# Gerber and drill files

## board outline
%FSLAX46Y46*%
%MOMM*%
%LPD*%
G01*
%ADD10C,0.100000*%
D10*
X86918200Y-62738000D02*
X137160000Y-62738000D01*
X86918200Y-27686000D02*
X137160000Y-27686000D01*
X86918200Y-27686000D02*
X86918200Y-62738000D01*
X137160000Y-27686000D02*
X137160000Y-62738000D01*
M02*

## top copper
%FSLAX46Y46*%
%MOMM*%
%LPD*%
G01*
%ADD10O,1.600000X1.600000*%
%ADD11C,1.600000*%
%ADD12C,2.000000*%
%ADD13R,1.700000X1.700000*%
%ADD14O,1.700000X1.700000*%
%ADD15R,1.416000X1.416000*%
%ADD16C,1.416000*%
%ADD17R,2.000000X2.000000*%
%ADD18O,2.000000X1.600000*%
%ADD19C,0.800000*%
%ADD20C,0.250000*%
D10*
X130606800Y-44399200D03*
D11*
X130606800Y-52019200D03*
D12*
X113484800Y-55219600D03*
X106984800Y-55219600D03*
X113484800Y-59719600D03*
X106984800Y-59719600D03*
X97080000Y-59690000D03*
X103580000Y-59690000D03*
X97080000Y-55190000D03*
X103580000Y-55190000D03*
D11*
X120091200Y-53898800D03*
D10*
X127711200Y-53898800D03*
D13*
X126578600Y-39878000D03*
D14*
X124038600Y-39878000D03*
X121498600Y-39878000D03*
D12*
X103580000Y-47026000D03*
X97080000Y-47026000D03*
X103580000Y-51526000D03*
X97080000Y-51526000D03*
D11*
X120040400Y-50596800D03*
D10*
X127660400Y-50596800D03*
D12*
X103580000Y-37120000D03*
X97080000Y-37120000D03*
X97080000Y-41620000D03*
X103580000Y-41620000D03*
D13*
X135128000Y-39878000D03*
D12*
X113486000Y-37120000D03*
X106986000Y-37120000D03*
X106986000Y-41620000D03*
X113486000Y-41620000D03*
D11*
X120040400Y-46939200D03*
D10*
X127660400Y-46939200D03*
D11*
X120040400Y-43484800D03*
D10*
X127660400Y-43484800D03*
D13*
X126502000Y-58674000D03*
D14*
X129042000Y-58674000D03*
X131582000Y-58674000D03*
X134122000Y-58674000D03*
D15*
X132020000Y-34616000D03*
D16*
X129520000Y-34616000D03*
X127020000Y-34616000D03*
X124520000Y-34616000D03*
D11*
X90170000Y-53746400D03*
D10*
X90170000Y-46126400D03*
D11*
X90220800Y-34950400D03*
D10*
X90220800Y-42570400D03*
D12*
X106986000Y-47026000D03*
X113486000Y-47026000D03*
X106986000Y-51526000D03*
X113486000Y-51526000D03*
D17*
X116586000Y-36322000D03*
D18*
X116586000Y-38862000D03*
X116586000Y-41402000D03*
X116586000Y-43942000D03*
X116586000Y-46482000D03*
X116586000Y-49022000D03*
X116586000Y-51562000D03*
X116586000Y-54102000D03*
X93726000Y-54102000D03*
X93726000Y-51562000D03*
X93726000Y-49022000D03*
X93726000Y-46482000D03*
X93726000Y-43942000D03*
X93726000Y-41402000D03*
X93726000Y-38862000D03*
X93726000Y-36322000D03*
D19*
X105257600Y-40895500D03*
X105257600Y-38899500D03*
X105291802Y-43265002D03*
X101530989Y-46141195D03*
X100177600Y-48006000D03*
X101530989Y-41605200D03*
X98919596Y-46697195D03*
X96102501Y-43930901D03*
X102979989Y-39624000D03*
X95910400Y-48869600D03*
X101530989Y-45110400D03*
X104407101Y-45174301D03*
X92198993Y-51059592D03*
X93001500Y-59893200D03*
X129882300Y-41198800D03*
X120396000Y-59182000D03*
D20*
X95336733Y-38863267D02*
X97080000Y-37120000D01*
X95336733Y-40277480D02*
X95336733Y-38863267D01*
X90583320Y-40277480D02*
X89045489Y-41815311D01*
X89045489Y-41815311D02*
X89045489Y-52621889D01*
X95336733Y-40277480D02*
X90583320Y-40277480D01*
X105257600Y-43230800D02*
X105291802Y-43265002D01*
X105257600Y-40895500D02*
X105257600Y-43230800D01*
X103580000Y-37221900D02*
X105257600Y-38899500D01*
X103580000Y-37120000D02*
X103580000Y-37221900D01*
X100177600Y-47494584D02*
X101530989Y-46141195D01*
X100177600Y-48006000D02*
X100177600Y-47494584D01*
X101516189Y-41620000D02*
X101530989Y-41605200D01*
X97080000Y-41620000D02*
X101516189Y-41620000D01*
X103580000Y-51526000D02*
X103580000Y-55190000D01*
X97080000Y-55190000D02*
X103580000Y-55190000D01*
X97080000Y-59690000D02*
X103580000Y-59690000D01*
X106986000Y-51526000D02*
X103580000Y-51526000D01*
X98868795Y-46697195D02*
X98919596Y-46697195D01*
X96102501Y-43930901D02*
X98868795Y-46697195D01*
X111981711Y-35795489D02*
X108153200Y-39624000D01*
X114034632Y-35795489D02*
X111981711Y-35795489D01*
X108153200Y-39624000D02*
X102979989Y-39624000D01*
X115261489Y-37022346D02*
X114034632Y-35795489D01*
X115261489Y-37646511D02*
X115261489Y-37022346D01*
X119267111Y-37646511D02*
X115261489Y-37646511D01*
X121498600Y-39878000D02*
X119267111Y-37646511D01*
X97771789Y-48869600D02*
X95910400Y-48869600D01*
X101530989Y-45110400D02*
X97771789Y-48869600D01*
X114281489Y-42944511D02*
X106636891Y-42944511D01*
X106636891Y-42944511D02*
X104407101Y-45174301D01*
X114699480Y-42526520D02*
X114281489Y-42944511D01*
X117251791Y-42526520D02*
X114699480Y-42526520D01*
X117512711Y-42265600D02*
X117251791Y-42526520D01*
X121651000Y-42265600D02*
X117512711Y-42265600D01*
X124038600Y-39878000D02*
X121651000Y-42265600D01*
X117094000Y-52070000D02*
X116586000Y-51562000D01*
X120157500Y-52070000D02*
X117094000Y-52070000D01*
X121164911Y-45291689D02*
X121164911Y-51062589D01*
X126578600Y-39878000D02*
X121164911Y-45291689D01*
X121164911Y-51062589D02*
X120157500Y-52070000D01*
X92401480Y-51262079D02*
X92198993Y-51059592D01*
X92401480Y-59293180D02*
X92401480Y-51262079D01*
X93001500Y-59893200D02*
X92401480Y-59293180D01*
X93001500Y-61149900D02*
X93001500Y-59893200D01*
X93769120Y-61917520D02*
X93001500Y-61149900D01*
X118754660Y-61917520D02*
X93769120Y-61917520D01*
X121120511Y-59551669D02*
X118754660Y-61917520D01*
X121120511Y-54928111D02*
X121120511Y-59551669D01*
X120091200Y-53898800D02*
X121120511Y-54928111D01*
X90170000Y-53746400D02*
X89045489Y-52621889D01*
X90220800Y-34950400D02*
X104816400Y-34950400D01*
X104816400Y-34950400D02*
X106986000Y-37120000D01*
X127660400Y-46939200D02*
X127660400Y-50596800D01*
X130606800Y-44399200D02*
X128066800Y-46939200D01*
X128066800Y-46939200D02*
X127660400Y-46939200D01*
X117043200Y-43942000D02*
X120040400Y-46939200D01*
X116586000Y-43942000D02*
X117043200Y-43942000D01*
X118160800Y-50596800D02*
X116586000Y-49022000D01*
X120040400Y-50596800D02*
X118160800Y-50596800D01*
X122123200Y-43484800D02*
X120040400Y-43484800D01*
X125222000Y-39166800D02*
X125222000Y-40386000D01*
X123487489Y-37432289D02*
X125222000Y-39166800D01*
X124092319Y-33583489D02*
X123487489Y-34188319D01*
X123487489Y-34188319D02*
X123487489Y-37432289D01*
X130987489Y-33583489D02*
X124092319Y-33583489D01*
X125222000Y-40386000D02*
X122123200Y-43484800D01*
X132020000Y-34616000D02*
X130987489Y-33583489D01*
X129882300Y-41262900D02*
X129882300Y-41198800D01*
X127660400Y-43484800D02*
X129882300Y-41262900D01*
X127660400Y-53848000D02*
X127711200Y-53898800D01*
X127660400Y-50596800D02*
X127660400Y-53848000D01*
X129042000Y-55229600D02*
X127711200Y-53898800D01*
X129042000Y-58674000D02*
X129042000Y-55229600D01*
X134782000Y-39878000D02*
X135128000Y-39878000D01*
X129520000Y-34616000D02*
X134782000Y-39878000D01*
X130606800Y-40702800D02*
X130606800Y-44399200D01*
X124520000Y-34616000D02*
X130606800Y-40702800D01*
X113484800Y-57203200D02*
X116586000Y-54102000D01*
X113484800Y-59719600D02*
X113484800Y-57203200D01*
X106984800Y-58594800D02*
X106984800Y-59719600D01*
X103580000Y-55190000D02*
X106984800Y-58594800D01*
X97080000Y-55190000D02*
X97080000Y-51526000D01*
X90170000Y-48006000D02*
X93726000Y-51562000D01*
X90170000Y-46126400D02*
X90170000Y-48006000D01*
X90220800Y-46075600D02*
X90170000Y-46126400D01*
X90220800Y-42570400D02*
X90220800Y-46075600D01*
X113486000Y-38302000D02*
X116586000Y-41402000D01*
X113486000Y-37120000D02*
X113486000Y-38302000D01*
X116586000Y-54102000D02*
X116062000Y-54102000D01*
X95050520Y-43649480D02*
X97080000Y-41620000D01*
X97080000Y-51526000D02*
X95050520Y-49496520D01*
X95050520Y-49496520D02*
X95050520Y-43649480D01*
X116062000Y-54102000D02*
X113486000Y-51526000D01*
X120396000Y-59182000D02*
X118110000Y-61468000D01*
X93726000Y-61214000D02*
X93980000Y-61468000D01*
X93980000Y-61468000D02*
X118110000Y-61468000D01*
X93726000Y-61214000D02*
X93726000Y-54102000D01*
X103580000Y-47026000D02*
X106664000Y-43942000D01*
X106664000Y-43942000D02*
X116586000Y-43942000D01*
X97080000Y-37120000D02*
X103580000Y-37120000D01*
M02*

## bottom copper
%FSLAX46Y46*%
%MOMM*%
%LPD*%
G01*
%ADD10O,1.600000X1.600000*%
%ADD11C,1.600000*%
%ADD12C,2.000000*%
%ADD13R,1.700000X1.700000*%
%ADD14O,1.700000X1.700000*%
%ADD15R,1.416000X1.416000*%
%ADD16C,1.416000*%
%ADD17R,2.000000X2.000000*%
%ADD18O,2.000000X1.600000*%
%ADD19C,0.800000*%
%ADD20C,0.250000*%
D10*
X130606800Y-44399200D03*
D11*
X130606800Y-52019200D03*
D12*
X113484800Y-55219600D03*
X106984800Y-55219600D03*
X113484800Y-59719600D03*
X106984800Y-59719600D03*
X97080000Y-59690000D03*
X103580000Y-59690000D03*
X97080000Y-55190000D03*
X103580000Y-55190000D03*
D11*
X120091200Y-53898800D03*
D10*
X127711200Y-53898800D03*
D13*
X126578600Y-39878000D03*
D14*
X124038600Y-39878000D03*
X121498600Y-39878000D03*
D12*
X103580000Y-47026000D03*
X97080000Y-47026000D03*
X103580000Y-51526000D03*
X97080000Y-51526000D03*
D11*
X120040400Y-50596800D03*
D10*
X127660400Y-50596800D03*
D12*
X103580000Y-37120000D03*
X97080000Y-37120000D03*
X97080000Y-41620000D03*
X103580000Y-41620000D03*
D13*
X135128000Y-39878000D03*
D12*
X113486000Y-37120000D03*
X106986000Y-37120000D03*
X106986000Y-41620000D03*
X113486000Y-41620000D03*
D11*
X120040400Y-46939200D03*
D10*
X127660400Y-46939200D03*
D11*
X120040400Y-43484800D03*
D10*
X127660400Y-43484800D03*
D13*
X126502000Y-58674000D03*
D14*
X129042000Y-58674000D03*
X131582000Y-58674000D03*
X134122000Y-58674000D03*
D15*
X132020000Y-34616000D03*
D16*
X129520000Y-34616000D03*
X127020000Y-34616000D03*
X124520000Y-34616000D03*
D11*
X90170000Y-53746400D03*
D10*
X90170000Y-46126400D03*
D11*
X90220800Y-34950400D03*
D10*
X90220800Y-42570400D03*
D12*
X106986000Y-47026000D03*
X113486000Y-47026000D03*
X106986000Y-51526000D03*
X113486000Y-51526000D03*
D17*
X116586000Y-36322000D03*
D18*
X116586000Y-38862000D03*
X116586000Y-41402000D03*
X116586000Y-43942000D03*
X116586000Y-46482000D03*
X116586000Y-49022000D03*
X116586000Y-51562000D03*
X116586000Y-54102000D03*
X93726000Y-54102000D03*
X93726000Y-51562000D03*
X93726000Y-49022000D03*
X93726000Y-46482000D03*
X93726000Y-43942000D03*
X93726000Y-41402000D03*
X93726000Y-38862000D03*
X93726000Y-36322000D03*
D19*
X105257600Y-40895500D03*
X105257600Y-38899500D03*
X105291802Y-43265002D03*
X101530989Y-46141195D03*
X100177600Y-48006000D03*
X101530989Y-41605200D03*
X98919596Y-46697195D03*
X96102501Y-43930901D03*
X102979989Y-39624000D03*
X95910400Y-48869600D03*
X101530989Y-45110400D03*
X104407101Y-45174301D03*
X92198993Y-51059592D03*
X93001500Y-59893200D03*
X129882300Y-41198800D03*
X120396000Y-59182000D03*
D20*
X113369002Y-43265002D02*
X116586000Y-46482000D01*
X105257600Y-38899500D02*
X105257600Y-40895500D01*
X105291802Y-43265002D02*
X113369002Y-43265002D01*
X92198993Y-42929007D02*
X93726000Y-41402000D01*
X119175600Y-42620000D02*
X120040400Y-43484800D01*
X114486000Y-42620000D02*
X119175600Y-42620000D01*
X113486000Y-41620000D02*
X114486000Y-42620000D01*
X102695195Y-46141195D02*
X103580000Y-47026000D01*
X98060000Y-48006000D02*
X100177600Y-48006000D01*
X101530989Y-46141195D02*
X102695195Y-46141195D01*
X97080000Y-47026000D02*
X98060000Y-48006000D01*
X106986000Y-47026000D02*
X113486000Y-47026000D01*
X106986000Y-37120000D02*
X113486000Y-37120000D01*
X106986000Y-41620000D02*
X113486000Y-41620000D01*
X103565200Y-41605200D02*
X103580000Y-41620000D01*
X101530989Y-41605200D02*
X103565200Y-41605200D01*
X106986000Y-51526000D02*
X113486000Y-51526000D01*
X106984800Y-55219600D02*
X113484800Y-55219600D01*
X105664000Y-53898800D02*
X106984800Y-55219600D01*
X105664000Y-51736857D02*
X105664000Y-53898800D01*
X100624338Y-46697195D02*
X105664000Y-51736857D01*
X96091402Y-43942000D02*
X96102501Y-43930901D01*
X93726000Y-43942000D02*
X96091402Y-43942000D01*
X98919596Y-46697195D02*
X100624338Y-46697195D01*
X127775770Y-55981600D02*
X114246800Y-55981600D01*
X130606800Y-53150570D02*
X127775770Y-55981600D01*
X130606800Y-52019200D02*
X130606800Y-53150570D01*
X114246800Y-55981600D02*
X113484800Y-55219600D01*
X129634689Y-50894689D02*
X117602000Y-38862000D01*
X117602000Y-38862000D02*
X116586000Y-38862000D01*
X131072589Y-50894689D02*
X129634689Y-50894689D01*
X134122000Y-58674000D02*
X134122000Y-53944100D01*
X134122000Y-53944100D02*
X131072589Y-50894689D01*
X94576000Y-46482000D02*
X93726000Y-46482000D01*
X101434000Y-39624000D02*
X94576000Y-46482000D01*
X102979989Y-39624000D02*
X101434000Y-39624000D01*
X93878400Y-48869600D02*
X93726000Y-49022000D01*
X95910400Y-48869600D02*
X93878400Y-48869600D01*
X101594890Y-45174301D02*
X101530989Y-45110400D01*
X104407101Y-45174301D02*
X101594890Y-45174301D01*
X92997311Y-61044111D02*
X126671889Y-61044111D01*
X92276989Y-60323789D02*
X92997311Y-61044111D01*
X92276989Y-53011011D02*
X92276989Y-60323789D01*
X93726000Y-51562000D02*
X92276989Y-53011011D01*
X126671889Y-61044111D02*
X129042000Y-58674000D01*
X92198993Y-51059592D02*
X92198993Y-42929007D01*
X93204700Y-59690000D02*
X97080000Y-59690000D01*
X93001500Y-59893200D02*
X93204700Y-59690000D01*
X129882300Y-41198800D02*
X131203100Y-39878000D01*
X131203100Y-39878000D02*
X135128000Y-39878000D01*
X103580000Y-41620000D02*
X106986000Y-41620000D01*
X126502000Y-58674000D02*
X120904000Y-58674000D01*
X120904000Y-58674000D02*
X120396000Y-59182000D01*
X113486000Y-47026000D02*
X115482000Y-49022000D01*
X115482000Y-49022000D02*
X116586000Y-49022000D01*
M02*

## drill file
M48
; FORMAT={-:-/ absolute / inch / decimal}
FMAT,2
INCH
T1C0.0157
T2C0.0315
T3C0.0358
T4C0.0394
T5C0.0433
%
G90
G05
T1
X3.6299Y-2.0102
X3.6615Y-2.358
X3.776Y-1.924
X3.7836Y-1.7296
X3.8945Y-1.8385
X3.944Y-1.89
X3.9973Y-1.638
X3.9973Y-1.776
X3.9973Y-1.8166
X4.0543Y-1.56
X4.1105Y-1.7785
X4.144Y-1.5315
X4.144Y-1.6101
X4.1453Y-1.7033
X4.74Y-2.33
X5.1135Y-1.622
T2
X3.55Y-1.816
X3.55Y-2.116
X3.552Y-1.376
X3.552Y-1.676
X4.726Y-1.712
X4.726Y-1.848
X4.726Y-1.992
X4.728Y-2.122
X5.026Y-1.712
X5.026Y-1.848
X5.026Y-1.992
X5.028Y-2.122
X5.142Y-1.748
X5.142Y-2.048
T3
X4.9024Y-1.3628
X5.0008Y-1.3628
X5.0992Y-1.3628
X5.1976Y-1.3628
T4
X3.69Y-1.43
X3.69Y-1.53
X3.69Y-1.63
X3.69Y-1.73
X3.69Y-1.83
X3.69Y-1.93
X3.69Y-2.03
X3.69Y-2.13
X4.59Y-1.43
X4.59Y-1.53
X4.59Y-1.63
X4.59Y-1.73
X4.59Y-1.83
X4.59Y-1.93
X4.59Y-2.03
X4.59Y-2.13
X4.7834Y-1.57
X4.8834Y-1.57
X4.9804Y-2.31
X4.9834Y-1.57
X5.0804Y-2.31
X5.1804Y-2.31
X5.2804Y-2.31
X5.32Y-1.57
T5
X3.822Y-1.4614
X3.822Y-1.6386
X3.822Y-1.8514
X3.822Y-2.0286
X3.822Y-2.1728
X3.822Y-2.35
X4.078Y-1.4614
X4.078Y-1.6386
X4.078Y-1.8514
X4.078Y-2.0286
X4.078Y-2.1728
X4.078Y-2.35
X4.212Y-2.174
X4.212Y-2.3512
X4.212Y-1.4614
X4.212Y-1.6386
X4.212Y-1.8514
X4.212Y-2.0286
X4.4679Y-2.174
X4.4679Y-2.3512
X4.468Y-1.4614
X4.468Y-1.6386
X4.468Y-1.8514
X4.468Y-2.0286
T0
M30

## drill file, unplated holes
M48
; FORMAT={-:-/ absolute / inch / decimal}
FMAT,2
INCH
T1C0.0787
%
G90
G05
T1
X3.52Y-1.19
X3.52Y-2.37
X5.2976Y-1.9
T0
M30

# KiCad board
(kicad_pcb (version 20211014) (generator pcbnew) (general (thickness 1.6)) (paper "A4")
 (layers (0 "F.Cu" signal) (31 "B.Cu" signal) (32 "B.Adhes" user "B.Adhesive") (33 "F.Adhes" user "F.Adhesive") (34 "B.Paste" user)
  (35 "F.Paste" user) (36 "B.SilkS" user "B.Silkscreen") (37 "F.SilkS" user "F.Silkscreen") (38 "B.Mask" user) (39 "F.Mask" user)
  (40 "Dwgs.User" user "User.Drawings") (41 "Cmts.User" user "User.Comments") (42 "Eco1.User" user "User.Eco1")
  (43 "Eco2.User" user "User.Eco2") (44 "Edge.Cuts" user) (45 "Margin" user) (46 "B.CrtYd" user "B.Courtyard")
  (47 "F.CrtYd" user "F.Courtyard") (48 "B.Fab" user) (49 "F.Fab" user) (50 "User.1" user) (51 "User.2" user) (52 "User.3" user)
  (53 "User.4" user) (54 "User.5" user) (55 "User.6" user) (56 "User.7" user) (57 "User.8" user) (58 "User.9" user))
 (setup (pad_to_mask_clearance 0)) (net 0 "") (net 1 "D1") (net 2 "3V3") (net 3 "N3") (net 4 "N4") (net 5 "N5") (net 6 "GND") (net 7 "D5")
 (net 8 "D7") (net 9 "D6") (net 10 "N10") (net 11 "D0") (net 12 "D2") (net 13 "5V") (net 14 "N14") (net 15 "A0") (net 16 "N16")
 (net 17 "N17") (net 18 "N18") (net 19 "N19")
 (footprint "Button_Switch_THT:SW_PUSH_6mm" (layer "F.Cu") (at 103.58 59.69 180)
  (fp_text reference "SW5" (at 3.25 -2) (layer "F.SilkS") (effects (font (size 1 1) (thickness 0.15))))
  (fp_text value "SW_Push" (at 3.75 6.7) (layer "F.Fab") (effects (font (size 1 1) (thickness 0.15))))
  (pad "1" thru_hole circle (at 0 0 270) (size 2 2) (drill 1.1) (layers *.Cu *.Mask) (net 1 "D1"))
  (pad "1" thru_hole circle (at 6.5 0 270) (size 2 2) (drill 1.1) (layers *.Cu *.Mask) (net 1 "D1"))
  (pad "2" thru_hole circle (at 6.5 4.5 270) (size 2 2) (drill 1.1) (layers *.Cu *.Mask) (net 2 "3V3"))
  (pad "2" thru_hole circle (at 0 4.5 270) (size 2 2) (drill 1.1) (layers *.Cu *.Mask) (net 2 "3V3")))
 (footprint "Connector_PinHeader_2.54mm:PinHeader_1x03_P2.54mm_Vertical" (layer "F.Cu") (at 126.5786 39.878 -90)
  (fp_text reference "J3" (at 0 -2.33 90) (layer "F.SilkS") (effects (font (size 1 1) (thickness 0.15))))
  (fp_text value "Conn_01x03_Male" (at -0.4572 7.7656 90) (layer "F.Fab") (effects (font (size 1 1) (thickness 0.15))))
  (pad "1" thru_hole rect (at 0 0 270) (size 1.7 1.7) (drill 1) (layers *.Cu *.Mask) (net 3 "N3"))
  (pad "2" thru_hole oval (at 0 2.54 270) (size 1.7 1.7) (drill 1) (layers *.Cu *.Mask) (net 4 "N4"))
  (pad "3" thru_hole oval (at 0 5.08 270) (size 1.7 1.7) (drill 1) (layers *.Cu *.Mask) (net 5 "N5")))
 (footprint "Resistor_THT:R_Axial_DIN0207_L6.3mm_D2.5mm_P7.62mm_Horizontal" (layer "F.Cu") (at 120.0912 53.8988)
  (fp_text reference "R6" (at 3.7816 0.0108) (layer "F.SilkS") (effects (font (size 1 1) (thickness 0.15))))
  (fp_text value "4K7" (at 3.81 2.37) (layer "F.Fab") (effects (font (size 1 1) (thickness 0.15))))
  (pad "1" thru_hole circle (at 0 0) (size 1.6 1.6) (drill 0.8) (layers *.Cu *.Mask) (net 1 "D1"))
  (pad "2" thru_hole oval (at 7.62 0) (size 1.6 1.6) (drill 0.8) (layers *.Cu *.Mask) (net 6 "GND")))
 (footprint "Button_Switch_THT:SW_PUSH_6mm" (layer "F.Cu") (at 97.08 47.026)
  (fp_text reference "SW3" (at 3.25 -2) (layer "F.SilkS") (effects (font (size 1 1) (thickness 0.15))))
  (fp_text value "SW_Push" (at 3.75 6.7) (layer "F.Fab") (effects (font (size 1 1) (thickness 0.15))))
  (pad "1" thru_hole circle (at 6.5 0 90) (size 2 2) (drill 1.1) (layers *.Cu *.Mask) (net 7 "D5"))
  (pad "1" thru_hole circle (at 0 0 90) (size 2 2) (drill 1.1) (layers *.Cu *.Mask) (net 7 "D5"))
  (pad "2" thru_hole circle (at 6.5 4.5 90) (size 2 2) (drill 1.1) (layers *.Cu *.Mask) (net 2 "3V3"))
  (pad "2" thru_hole circle (at 0 4.5 90) (size 2 2) (drill 1.1) (layers *.Cu *.Mask) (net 2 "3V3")))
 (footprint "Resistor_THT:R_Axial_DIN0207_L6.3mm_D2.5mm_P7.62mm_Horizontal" (layer "F.Cu") (at 120.0404 50.5968)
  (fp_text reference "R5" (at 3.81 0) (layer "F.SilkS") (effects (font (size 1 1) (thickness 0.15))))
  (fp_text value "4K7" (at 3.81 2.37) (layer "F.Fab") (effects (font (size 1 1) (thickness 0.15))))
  (pad "1" thru_hole circle (at 0 0) (size 1.6 1.6) (drill 0.8) (layers *.Cu *.Mask) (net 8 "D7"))
  (pad "2" thru_hole oval (at 7.62 0) (size 1.6 1.6) (drill 0.8) (layers *.Cu *.Mask) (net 6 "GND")))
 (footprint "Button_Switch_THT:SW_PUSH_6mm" (layer "F.Cu") (at 97.08 37.12)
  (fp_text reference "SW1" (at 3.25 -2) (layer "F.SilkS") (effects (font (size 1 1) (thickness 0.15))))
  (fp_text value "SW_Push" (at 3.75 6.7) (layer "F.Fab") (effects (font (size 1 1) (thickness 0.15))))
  (pad "1" thru_hole circle (at 6.5 0 90) (size 2 2) (drill 1.1) (layers *.Cu *.Mask) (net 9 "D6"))
  (pad "1" thru_hole circle (at 0 0 90) (size 2 2) (drill 1.1) (layers *.Cu *.Mask) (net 9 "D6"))
  (pad "2" thru_hole circle (at 0 4.5 90) (size 2 2) (drill 1.1) (layers *.Cu *.Mask) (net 2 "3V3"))
  (pad "2" thru_hole circle (at 6.5 4.5 90) (size 2 2) (drill 1.1) (layers *.Cu *.Mask) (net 2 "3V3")))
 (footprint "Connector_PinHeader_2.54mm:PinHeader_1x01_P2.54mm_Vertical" (layer "F.Cu") (at 135.128 39.878)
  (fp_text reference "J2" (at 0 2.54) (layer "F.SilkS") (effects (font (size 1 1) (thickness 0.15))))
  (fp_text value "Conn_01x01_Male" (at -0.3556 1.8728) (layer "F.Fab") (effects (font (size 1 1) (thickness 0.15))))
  (pad "1" thru_hole rect (at 0 0) (size 1.7 1.7) (drill 1) (layers *.Cu *.Mask) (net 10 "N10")))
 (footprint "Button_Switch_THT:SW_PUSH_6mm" (layer "F.Cu") (at 106.986 37.12)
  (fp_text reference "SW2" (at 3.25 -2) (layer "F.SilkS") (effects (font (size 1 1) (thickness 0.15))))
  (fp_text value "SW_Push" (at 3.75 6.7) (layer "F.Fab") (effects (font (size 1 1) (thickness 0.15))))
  (pad "1" thru_hole circle (at 6.5 0 90) (size 2 2) (drill 1.1) (layers *.Cu *.Mask) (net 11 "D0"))
  (pad "1" thru_hole circle (at 0 0 90) (size 2 2) (drill 1.1) (layers *.Cu *.Mask) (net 11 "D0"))
  (pad "2" thru_hole circle (at 0 4.5 90) (size 2 2) (drill 1.1) (layers *.Cu *.Mask) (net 2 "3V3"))
  (pad "2" thru_hole circle (at 6.5 4.5 90) (size 2 2) (drill 1.1) (layers *.Cu *.Mask) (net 2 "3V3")))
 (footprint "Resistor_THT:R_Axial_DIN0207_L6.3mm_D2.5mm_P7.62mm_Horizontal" (layer "F.Cu") (at 130.6068 52.0192 90)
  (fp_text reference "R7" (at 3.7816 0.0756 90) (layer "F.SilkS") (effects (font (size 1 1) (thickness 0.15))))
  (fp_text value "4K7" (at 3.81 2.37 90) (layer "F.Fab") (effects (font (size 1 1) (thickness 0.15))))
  (pad "1" thru_hole circle (at 0 0 90) (size 1.6 1.6) (drill 0.8) (layers *.Cu *.Mask) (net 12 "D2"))
  (pad "2" thru_hole oval (at 7.62 0 90) (size 1.6 1.6) (drill 0.8) (layers *.Cu *.Mask) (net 6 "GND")))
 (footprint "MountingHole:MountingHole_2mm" (layer "F.Cu") (at 89.408 60.198)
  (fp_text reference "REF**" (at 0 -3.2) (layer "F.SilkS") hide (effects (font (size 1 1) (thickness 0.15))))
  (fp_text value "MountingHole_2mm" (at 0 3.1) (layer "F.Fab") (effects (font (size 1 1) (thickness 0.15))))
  (pad "" np_thru_hole circle (at 0 0) (size 2 2) (drill 2) (layers *.Cu *.Mask)))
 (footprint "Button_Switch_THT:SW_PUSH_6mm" (layer "F.Cu") (at 106.9848 55.2196)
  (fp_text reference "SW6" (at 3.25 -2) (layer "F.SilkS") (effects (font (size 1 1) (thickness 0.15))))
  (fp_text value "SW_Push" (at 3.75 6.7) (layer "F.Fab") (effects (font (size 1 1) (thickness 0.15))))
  (pad "1" thru_hole circle (at 0 0 90) (size 2 2) (drill 1.1) (layers *.Cu *.Mask) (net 12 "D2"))
  (pad "1" thru_hole circle (at 6.5 0 90) (size 2 2) (drill 1.1) (layers *.Cu *.Mask) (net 12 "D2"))
  (pad "2" thru_hole circle (at 6.5 4.5 90) (size 2 2) (drill 1.1) (layers *.Cu *.Mask) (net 2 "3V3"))
  (pad "2" thru_hole circle (at 0 4.5 90) (size 2 2) (drill 1.1) (layers *.Cu *.Mask) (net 2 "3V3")))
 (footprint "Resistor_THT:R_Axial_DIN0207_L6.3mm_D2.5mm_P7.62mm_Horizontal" (layer "F.Cu") (at 120.0404 46.9392)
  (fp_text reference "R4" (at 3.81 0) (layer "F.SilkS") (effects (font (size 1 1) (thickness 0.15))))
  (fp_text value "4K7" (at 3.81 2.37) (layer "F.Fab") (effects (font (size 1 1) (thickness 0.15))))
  (pad "1" thru_hole circle (at 0 0) (size 1.6 1.6) (drill 0.8) (layers *.Cu *.Mask) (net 7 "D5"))
  (pad "2" thru_hole oval (at 7.62 0) (size 1.6 1.6) (drill 0.8) (layers *.Cu *.Mask) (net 6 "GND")))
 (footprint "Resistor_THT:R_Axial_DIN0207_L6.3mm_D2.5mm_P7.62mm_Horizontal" (layer "F.Cu") (at 120.0404 43.4848)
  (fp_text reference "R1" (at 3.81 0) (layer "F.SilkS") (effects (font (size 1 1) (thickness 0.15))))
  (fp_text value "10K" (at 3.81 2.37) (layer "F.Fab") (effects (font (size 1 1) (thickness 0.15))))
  (pad "1" thru_hole circle (at 0 0) (size 1.6 1.6) (drill 0.8) (layers *.Cu *.Mask) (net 2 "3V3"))
  (pad "2" thru_hole oval (at 7.62 0) (size 1.6 1.6) (drill 0.8) (layers *.Cu *.Mask) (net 10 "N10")))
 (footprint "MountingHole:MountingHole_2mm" (layer "F.Cu") (at 89.408 30.226)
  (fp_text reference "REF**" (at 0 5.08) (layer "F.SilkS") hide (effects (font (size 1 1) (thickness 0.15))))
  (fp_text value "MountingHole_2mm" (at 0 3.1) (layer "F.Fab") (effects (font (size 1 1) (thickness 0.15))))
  (pad "" np_thru_hole circle (at 0 0) (size 2 2) (drill 2) (layers *.Cu *.Mask)))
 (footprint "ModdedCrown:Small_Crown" (layer "F.Cu") (at 97.9424 30.3276)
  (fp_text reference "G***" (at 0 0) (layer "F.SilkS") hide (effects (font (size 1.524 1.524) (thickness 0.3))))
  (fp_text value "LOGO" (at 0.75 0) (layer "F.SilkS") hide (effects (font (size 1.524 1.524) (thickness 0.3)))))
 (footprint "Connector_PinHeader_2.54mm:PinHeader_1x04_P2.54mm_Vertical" (layer "F.Cu") (at 126.502 58.674 90)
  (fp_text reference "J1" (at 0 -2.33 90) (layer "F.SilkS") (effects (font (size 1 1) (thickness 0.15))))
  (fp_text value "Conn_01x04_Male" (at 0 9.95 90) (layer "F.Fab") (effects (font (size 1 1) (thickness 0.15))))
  (pad "1" thru_hole rect (at 0 0 90) (size 1.7 1.7) (drill 1) (layers *.Cu *.Mask) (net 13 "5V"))
  (pad "2" thru_hole oval (at 0 2.54 90) (size 1.7 1.7) (drill 1) (layers *.Cu *.Mask) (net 6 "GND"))
  (pad "3" thru_hole oval (at 0 5.08 90) (size 1.7 1.7) (drill 1) (layers *.Cu *.Mask) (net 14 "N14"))
  (pad "4" thru_hole oval (at 0 7.62 90) (size 1.7 1.7) (drill 1) (layers *.Cu *.Mask) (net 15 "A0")))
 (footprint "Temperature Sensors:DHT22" (layer "F.Cu") (at 132.02 34.616 180)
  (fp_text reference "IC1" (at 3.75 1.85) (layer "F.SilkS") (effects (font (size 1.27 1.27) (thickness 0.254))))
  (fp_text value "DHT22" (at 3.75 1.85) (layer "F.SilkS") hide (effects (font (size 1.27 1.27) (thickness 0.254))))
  (pad "1" thru_hole rect locked (at 0 0 180) (size 1.416 1.416) (drill 0.91) (layers *.Cu *.Mask) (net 2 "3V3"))
  (pad "2" thru_hole circle locked (at 2.5 0 180) (size 1.416 1.416) (drill 0.91) (layers *.Cu *.Mask) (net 10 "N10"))
  (pad "3" thru_hole circle locked (at 5 0 180) (size 1.416 1.416) (drill 0.91) (layers *.Cu *.Mask) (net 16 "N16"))
  (pad "4" thru_hole circle locked (at 7.5 0 180) (size 1.416 1.416) (drill 0.91) (layers *.Cu *.Mask) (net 6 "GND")))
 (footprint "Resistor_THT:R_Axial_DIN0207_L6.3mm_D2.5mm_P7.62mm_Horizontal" (layer "F.Cu") (at 90.17 53.7464 90)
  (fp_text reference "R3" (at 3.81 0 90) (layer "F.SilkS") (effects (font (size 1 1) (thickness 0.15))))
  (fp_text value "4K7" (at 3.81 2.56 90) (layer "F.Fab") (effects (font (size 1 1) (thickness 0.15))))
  (pad "1" thru_hole circle (at 0 0 90) (size 1.6 1.6) (drill 0.8) (layers *.Cu *.Mask) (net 9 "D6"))
  (pad "2" thru_hole oval (at 7.62 0 90) (size 1.6 1.6) (drill 0.8) (layers *.Cu *.Mask) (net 6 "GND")))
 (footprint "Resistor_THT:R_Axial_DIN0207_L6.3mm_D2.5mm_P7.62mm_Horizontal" (layer "F.Cu") (at 90.2208 34.9504 -90)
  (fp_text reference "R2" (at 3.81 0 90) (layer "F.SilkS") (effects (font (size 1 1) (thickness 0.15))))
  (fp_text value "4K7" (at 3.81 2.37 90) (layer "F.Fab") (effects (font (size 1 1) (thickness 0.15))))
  (pad "1" thru_hole circle (at 0 0 270) (size 1.6 1.6) (drill 0.8) (layers *.Cu *.Mask) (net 11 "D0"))
  (pad "2" thru_hole oval (at 7.62 0 270) (size 1.6 1.6) (drill 0.8) (layers *.Cu *.Mask) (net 6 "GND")))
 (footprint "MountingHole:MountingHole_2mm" (layer "F.Cu") (at 134.558 48.26)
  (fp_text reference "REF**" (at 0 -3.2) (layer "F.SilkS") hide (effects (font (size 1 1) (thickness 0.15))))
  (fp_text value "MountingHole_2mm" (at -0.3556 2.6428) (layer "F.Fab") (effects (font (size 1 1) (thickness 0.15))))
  (pad "" np_thru_hole circle (at 0 0) (size 2 2) (drill 2) (layers *.Cu *.Mask)))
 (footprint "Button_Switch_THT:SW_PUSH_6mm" (layer "F.Cu") (at 106.986 47.026)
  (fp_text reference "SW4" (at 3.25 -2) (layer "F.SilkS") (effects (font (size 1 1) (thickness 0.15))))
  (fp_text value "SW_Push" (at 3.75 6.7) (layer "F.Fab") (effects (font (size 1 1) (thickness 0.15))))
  (pad "1" thru_hole circle (at 0 0 90) (size 2 2) (drill 1.1) (layers *.Cu *.Mask) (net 8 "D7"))
  (pad "1" thru_hole circle (at 6.5 0 90) (size 2 2) (drill 1.1) (layers *.Cu *.Mask) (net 8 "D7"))
  (pad "2" thru_hole circle (at 0 4.5 90) (size 2 2) (drill 1.1) (layers *.Cu *.Mask) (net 2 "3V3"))
  (pad "2" thru_hole circle (at 6.5 4.5 90) (size 2 2) (drill 1.1) (layers *.Cu *.Mask) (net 2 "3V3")))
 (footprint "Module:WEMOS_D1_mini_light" (layer "B.Cu") (at 116.586 36.322 180)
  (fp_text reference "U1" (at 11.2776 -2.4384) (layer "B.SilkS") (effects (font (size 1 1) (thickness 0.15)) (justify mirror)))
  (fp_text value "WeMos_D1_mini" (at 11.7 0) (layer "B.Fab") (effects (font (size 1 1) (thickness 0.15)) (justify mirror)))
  (pad "1" thru_hole rect (at 0 0 180) (size 2 2) (drill 1) (layers *.Cu *.Mask) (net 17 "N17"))
  (pad "2" thru_hole oval (at 0 -2.54 180) (size 2 1.6) (drill 1) (layers *.Cu *.Mask) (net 15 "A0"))
  (pad "3" thru_hole oval (at 0 -5.08 180) (size 2 1.6) (drill 1) (layers *.Cu *.Mask) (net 11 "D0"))
  (pad "4" thru_hole oval (at 0 -7.62 180) (size 2 1.6) (drill 1) (layers *.Cu *.Mask) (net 7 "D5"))
  (pad "5" thru_hole oval (at 0 -10.16 180) (size 2 1.6) (drill 1) (layers *.Cu *.Mask) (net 9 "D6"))
  (pad "6" thru_hole oval (at 0 -12.7 180) (size 2 1.6) (drill 1) (layers *.Cu *.Mask) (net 8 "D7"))
  (pad "7" thru_hole oval (at 0 -15.24 180) (size 2 1.6) (drill 1) (layers *.Cu *.Mask) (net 3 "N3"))
  (pad "8" thru_hole oval (at 0 -17.78 180) (size 2 1.6) (drill 1) (layers *.Cu *.Mask) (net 2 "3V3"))
  (pad "9" thru_hole oval (at 22.86 -17.78 180) (size 2 1.6) (drill 1) (layers *.Cu *.Mask) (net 13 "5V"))
  (pad "10" thru_hole oval (at 22.86 -15.24 180) (size 2 1.6) (drill 1) (layers *.Cu *.Mask) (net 6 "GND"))
  (pad "11" thru_hole oval (at 22.86 -12.7 180) (size 2 1.6) (drill 1) (layers *.Cu *.Mask) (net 4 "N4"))
  (pad "12" thru_hole oval (at 22.86 -10.16 180) (size 2 1.6) (drill 1) (layers *.Cu *.Mask) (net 5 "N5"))
  (pad "13" thru_hole oval (at 22.86 -7.62 180) (size 2 1.6) (drill 1) (layers *.Cu *.Mask) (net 12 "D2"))
  (pad "14" thru_hole oval (at 22.86 -5.08 180) (size 2 1.6) (drill 1) (layers *.Cu *.Mask) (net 1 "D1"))
  (pad "15" thru_hole oval (at 22.86 -2.54 180) (size 2 1.6) (drill 1) (layers *.Cu *.Mask) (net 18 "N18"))
  (pad "16" thru_hole oval (at 22.86 0 180) (size 2 1.6) (drill 1) (layers *.Cu *.Mask) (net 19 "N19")))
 (gr_line (start 86.9182 62.738) (end 137.16 62.738) (layer "Edge.Cuts") (width 0.1))
 (gr_line (start 86.9182 27.686) (end 137.16 27.686) (layer "Edge.Cuts") (width 0.1))
 (gr_line (start 86.9182 27.686) (end 86.9182 62.738) (layer "Edge.Cuts") (width 0.1))
 (gr_line (start 137.16 27.686) (end 137.16 62.738) (layer "Edge.Cuts") (width 0.1))
 (segment (start 97.08 41.62) (end 101.516189 41.62) (width 0.25) (layer "F.Cu") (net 2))
 (segment (start 124.092319 33.583489) (end 123.487489 34.188319) (width 0.25) (layer "F.Cu") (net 2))
 (segment (start 113.4848 59.7196) (end 113.4848 57.2032) (width 0.25) (layer "F.Cu") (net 2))
 (segment (start 123.487489 34.188319) (end 123.487489 37.432289) (width 0.25) (layer "F.Cu") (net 2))
 (segment (start 132.02 34.616) (end 130.987489 33.583489) (width 0.25) (layer "F.Cu") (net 2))
 (segment (start 116.586 54.102) (end 116.062 54.102) (width 0.25) (layer "F.Cu") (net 2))
 (segment (start 101.516189 41.62) (end 101.530989 41.6052) (width 0.25) (layer "F.Cu") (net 2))
 (segment (start 125.222 39.1668) (end 125.222 40.386) (width 0.25) (layer "F.Cu") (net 2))
 (segment (start 125.222 40.386) (end 122.1232 43.4848) (width 0.25) (layer "F.Cu") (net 2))
 (segment (start 95.05052 43.64948) (end 97.08 41.62) (width 0.25) (layer "F.Cu") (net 2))
 (segment (start 113.4848 57.2032) (end 116.586 54.102) (width 0.25) (layer "F.Cu") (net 2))
 (segment (start 130.987489 33.583489) (end 124.092319 33.583489) (width 0.25) (layer "F.Cu") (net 2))
 (segment (start 97.08 55.19) (end 103.58 55.19) (width 0.25) (layer "F.Cu") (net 2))
 (segment (start 97.08 55.19) (end 97.08 51.526) (width 0.25) (layer "F.Cu") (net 2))
 (segment (start 122.1232 43.4848) (end 120.0404 43.4848) (width 0.25) (layer "F.Cu") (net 2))
 (segment (start 123.487489 37.432289) (end 125.222 39.1668) (width 0.25) (layer "F.Cu") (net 2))
 (segment (start 106.986 51.526) (end 103.58 51.526) (width 0.25) (layer "F.Cu") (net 2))
 (segment (start 97.08 51.526) (end 95.05052 49.49652) (width 0.25) (layer "F.Cu") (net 2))
 (segment (start 95.05052 49.49652) (end 95.05052 43.64948) (width 0.25) (layer "F.Cu") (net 2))
 (segment (start 103.58 51.526) (end 103.58 55.19) (width 0.25) (layer "F.Cu") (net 2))
 (segment (start 116.062 54.102) (end 113.486 51.526) (width 0.25) (layer "F.Cu") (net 2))
 (segment (start 103.58 55.19) (end 106.9848 58.5948) (width 0.25) (layer "F.Cu") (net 2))
 (segment (start 106.9848 58.5948) (end 106.9848 59.7196) (width 0.25) (layer "F.Cu") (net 2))
 (via (at 101.530989 41.6052) (size 0.8) (drill 0.4) (layers "F.Cu" "B.Cu") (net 2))
 (segment (start 114.486 42.62) (end 119.1756 42.62) (width 0.25) (layer "B.Cu") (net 2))
 (segment (start 113.486 41.62) (end 114.486 42.62) (width 0.25) (layer "B.Cu") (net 2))
 (segment (start 106.986 51.526) (end 113.486 51.526) (width 0.25) (layer "B.Cu") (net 2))
 (segment (start 106.986 41.62) (end 113.486 41.62) (width 0.25) (layer "B.Cu") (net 2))
 (segment (start 103.5652 41.6052) (end 103.58 41.62) (width 0.25) (layer "B.Cu") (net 2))
 (segment (start 101.530989 41.6052) (end 103.5652 41.6052) (width 0.25) (layer "B.Cu") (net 2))
 (segment (start 119.1756 42.62) (end 120.0404 43.4848) (width 0.25) (layer "B.Cu") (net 2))
 (segment (start 103.58 41.62) (end 106.986 41.62) (width 0.25) (layer "B.Cu") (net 2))
 (segment (start 134.782 39.878) (end 135.128 39.878) (width 0.25) (layer "F.Cu") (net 10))
 (segment (start 129.52 34.616) (end 134.782 39.878) (width 0.25) (layer "F.Cu") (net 10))
 (segment (start 127.6604 43.4848) (end 129.8823 41.2629) (width 0.25) (layer "F.Cu") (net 10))
 (segment (start 129.8823 41.2629) (end 129.8823 41.1988) (width 0.25) (layer "F.Cu") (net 10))
 (via (at 129.8823 41.1988) (size 0.8) (drill 0.4) (layers "F.Cu" "B.Cu") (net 10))
 (segment (start 131.2031 39.878) (end 135.128 39.878) (width 0.25) (layer "B.Cu") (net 10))
 (segment (start 129.8823 41.1988) (end 131.2031 39.878) (width 0.25) (layer "B.Cu") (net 10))
 (segment (start 130.6068 44.3992) (end 128.0668 46.9392) (width 0.25) (layer "F.Cu") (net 6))
 (segment (start 90.2208 46.0756) (end 90.17 46.1264) (width 0.25) (layer "F.Cu") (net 6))
 (segment (start 130.6068 40.7028) (end 130.6068 44.3992) (width 0.25) (layer "F.Cu") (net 6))
 (segment (start 127.6604 53.848) (end 127.7112 53.8988) (width 0.25) (layer "F.Cu") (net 6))
 (segment (start 127.6604 50.5968) (end 127.6604 53.848) (width 0.25) (layer "F.Cu") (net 6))
 (segment (start 124.52 34.616) (end 130.6068 40.7028) (width 0.25) (layer "F.Cu") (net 6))
 (segment (start 127.6604 46.9392) (end 127.6604 50.5968) (width 0.25) (layer "F.Cu") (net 6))
 (segment (start 128.0668 46.9392) (end 127.6604 46.9392) (width 0.25) (layer "F.Cu") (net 6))
 (segment (start 90.2208 42.5704) (end 90.2208 46.0756) (width 0.25) (layer "F.Cu") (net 6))
 (segment (start 129.042 55.2296) (end 127.7112 53.8988) (width 0.25) (layer "F.Cu") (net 6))
 (segment (start 90.17 48.006) (end 93.726 51.562) (width 0.25) (layer "F.Cu") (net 6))
 (segment (start 90.17 46.1264) (end 90.17 48.006) (width 0.25) (layer "F.Cu") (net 6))
 (segment (start 129.042 58.674) (end 129.042 55.2296) (width 0.25) (layer "F.Cu") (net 6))
 (segment (start 93.726 51.562) (end 92.276989 53.011011) (width 0.25) (layer "B.Cu") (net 6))
 (segment (start 126.671889 61.044111) (end 129.042 58.674) (width 0.25) (layer "B.Cu") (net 6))
 (segment (start 92.997311 61.044111) (end 126.671889 61.044111) (width 0.25) (layer "B.Cu") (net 6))
 (segment (start 92.276989 53.011011) (end 92.276989 60.323789) (width 0.25) (layer "B.Cu") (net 6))
 (segment (start 92.276989 60.323789) (end 92.997311 61.044111) (width 0.25) (layer "B.Cu") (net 6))
 (segment (start 120.396 59.182) (end 118.11 61.468) (width 0.25) (layer "F.Cu") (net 13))
 (segment (start 93.726 61.214) (end 93.98 61.468) (width 0.25) (layer "F.Cu") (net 13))
 (segment (start 93.98 61.468) (end 118.11 61.468) (width 0.25) (layer "F.Cu") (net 13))
 (segment (start 93.726 61.214) (end 93.726 54.102) (width 0.25) (layer "F.Cu") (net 13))
 (via (at 120.396 59.182) (size 0.8) (drill 0.4) (layers "F.Cu" "B.Cu") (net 13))
 (segment (start 126.502 58.674) (end 120.904 58.674) (width 0.25) (layer "B.Cu") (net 13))
 (segment (start 120.904 58.674) (end 120.396 59.182) (width 0.25) (layer "B.Cu") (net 13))
 (segment (start 134.122 53.9441) (end 131.072589 50.894689) (width 0.25) (layer "B.Cu") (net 15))
 (segment (start 117.602 38.862) (end 116.586 38.862) (width 0.25) (layer "B.Cu") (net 15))
 (segment (start 134.122 58.674) (end 134.122 53.9441) (width 0.25) (layer "B.Cu") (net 15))
 (segment (start 129.634689 50.894689) (end 117.602 38.862) (width 0.25) (layer "B.Cu") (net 15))
 (segment (start 131.072589 50.894689) (end 129.634689 50.894689) (width 0.25) (layer "B.Cu") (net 15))
 (segment (start 121.164911 51.062589) (end 120.1575 52.07) (width 0.25) (layer "F.Cu") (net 3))
 (segment (start 117.094 52.07) (end 116.586 51.562) (width 0.25) (layer "F.Cu") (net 3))
 (segment (start 120.1575 52.07) (end 117.094 52.07) (width 0.25) (layer "F.Cu") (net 3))
 (segment (start 126.5786 39.878) (end 121.164911 45.291689) (width 0.25) (layer "F.Cu") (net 3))
 (segment (start 121.164911 45.291689) (end 121.164911 51.062589) (width 0.25) (layer "F.Cu") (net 3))
 (segment (start 106.636891 42.944511) (end 104.407101 45.174301) (width 0.25) (layer "F.Cu") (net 4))
 (segment (start 114.281489 42.944511) (end 106.636891 42.944511) (width 0.25) (layer "F.Cu") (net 4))
 (segment (start 101.530989 45.1104) (end 97.771789 48.8696) (width 0.25) (layer "F.Cu") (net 4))
 (segment (start 124.0386 39.878) (end 121.651 42.2656) (width 0.25) (layer "F.Cu") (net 4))
 (segment (start 117.251791 42.52652) (end 114.69948 42.52652) (width 0.25) (layer "F.Cu") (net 4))
 (segment (start 114.69948 42.52652) (end 114.281489 42.944511) (width 0.25) (layer "F.Cu") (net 4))
 (segment (start 117.512711 42.2656) (end 117.251791 42.52652) (width 0.25) (layer "F.Cu") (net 4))
 (segment (start 121.651 42.2656) (end 117.512711 42.2656) (width 0.25) (layer "F.Cu") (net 4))
 (segment (start 97.771789 48.8696) (end 95.9104 48.8696) (width 0.25) (layer "F.Cu") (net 4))
 (via (at 95.9104 48.8696) (size 0.8) (drill 0.4) (layers "F.Cu" "B.Cu") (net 4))
 (via (at 104.407101 45.174301) (size 0.8) (drill 0.4) (layers "F.Cu" "B.Cu") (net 4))
 (via (at 101.530989 45.1104) (size 0.8) (drill 0.4) (layers "F.Cu" "B.Cu") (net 4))
 (segment (start 93.8784 48.8696) (end 93.726 49.022) (width 0.25) (layer "B.Cu") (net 4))
 (segment (start 104.407101 45.174301) (end 101.59489 45.174301) (width 0.25) (layer "B.Cu") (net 4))
 (segment (start 101.59489 45.174301) (end 101.530989 45.1104) (width 0.25) (layer "B.Cu") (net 4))
 (segment (start 95.9104 48.8696) (end 93.8784 48.8696) (width 0.25) (layer "B.Cu") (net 4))
 (segment (start 115.261489 37.646511) (end 115.261489 37.022346) (width 0.25) (layer "F.Cu") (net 5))
 (segment (start 121.4986 39.878) (end 119.267111 37.646511) (width 0.25) (layer "F.Cu") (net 5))
 (segment (start 119.267111 37.646511) (end 115.261489 37.646511) (width 0.25) (layer "F.Cu") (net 5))
 (segment (start 111.981711 35.795489) (end 108.1532 39.624) (width 0.25) (layer "F.Cu") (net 5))
 (segment (start 108.1532 39.624) (end 102.979989 39.624) (width 0.25) (layer "F.Cu") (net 5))
 (segment (start 114.034632 35.795489) (end 111.981711 35.795489) (width 0.25) (layer "F.Cu") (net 5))
 (segment (start 115.261489 37.022346) (end 114.034632 35.795489) (width 0.25) (layer "F.Cu") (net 5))
 (via (at 102.979989 39.624) (size 0.8) (drill 0.4) (layers "F.Cu" "B.Cu") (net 5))
 (segment (start 94.576 46.482) (end 93.726 46.482) (width 0.25) (layer "B.Cu") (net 5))
 (segment (start 102.979989 39.624) (end 101.434 39.624) (width 0.25) (layer "B.Cu") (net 5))
 (segment (start 101.434 39.624) (end 94.576 46.482) (width 0.25) (layer "B.Cu") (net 5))
 (segment (start 113.486 38.302) (end 116.586 41.402) (width 0.25) (layer "F.Cu") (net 11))
 (segment (start 104.8164 34.9504) (end 106.986 37.12) (width 0.25) (layer "F.Cu") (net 11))
 (segment (start 90.2208 34.9504) (end 104.8164 34.9504) (width 0.25) (layer "F.Cu") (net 11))
 (segment (start 113.486 37.12) (end 113.486 38.302) (width 0.25) (layer "F.Cu") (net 11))
 (segment (start 106.986 37.12) (end 113.486 37.12) (width 0.25) (layer "B.Cu") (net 11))
 (segment (start 100.1776 47.494584) (end 101.530989 46.141195) (width 0.25) (layer "F.Cu") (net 7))
 (segment (start 103.58 47.026) (end 106.664 43.942) (width 0.25) (layer "F.Cu") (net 7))
 (segment (start 100.1776 48.006) (end 100.1776 47.494584) (width 0.25) (layer "F.Cu") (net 7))
 (segment (start 117.0432 43.942) (end 120.0404 46.9392) (width 0.25) (layer "F.Cu") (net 7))
 (segment (start 116.586 43.942) (end 117.0432 43.942) (width 0.25) (layer "F.Cu") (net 7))
 (segment (start 106.664 43.942) (end 116.586 43.942) (width 0.25) (layer "F.Cu") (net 7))
 (via (at 101.530989 46.141195) (size 0.8) (drill 0.4) (layers "F.Cu" "B.Cu") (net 7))
 (via (at 100.1776 48.006) (size 0.8) (drill 0.4) (layers "F.Cu" "B.Cu") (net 7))
 (segment (start 98.06 48.006) (end 100.1776 48.006) (width 0.25) (layer "B.Cu") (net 7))
 (segment (start 101.530989 46.141195) (end 102.695195 46.141195) (width 0.25) (layer "B.Cu") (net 7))
 (segment (start 97.08 47.026) (end 98.06 48.006) (width 0.25) (layer "B.Cu") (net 7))
 (segment (start 102.695195 46.141195) (end 103.58 47.026) (width 0.25) (layer "B.Cu") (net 7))
 (segment (start 105.2576 40.8955) (end 105.2576 43.2308) (width 0.25) (layer "F.Cu") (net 9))
 (segment (start 89.045489 41.815311) (end 89.045489 52.621889) (width 0.25) (layer "F.Cu") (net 9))
 (segment (start 103.58 37.2219) (end 105.2576 38.8995) (width 0.25) (layer "F.Cu") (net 9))
 (segment (start 97.08 37.12) (end 103.58 37.12) (width 0.25) (layer "F.Cu") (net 9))
 (segment (start 103.58 37.12) (end 103.58 37.2219) (width 0.25) (layer "F.Cu") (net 9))
 (segment (start 90.58332 40.27748) (end 89.045489 41.815311) (width 0.25) (layer "F.Cu") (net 9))
 (segment (start 105.2576 43.2308) (end 105.291802 43.265002) (width 0.25) (layer "F.Cu") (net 9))
 (segment (start 95.336733 40.27748) (end 95.336733 38.863267) (width 0.25) (layer "F.Cu") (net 9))
 (segment (start 95.336733 40.27748) (end 90.58332 40.27748) (width 0.25) (layer "F.Cu") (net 9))
 (segment (start 90.17 53.7464) (end 89.045489 52.621889) (width 0.25) (layer "F.Cu") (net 9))
 (segment (start 95.336733 38.863267) (end 97.08 37.12) (width 0.25) (layer "F.Cu") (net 9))
 (via (at 105.291802 43.265002) (size 0.8) (drill 0.4) (layers "F.Cu" "B.Cu") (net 9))
 (via (at 105.2576 38.8995) (size 0.8) (drill 0.4) (layers "F.Cu" "B.Cu") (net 9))
 (via (at 105.2576 40.8955) (size 0.8) (drill 0.4) (layers "F.Cu" "B.Cu") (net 9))
 (segment (start 113.369002 43.265002) (end 116.586 46.482) (width 0.25) (layer "B.Cu") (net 9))
 (segment (start 105.291802 43.265002) (end 113.369002 43.265002) (width 0.25) (layer "B.Cu") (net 9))
 (segment (start 105.2576 38.8995) (end 105.2576 40.8955) (width 0.25) (layer "B.Cu") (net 9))
 (segment (start 118.1608 50.5968) (end 116.586 49.022) (width 0.25) (layer "F.Cu") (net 8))
 (segment (start 120.0404 50.5968) (end 118.1608 50.5968) (width 0.25) (layer "F.Cu") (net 8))
 (segment (start 106.986 47.026) (end 113.486 47.026) (width 0.25) (layer "B.Cu") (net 8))
 (segment (start 113.486 47.026) (end 115.482 49.022) (width 0.25) (layer "B.Cu") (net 8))
 (segment (start 115.482 49.022) (end 116.586 49.022) (width 0.25) (layer "B.Cu") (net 8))
 (segment (start 121.120511 54.928111) (end 121.120511 59.551669) (width 0.25) (layer "F.Cu") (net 1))
 (segment (start 120.0912 53.8988) (end 121.120511 54.928111) (width 0.25) (layer "F.Cu") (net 1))
 (segment (start 93.76912 61.91752) (end 93.0015 61.1499) (width 0.25) (layer "F.Cu") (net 1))
 (segment (start 97.08 59.69) (end 103.58 59.69) (width 0.25) (layer "F.Cu") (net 1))
 (segment (start 92.40148 59.29318) (end 92.40148 51.262079) (width 0.25) (layer "F.Cu") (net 1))
 (segment (start 92.40148 51.262079) (end 92.198993 51.059592) (width 0.25) (layer "F.Cu") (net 1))
 (segment (start 118.75466 61.91752) (end 93.76912 61.91752) (width 0.25) (layer "F.Cu") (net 1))
 (segment (start 121.120511 59.551669) (end 118.75466 61.91752) (width 0.25) (layer "F.Cu") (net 1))
 (segment (start 93.0015 61.1499) (end 93.0015 59.8932) (width 0.25) (layer "F.Cu") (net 1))
 (segment (start 93.0015 59.8932) (end 92.40148 59.29318) (width 0.25) (layer "F.Cu") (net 1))
 (via (at 93.0015 59.8932) (size 0.8) (drill 0.4) (layers "F.Cu" "B.Cu") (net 1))
 (via (at 92.198993 51.059592) (size 0.8) (drill 0.4) (layers "F.Cu" "B.Cu") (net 1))
 (segment (start 93.2047 59.69) (end 97.08 59.69) (width 0.25) (layer "B.Cu") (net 1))
 (segment (start 93.0015 59.8932) (end 93.2047 59.69) (width 0.25) (layer "B.Cu") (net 1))
 (segment (start 92.198993 42.929007) (end 93.726 41.402) (width 0.25) (layer "B.Cu") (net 1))
 (segment (start 92.198993 51.059592) (end 92.198993 42.929007) (width 0.25) (layer "B.Cu") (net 1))
 (segment (start 98.868795 46.697195) (end 98.919596 46.697195) (width 0.25) (layer "F.Cu") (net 12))
 (segment (start 96.102501 43.930901) (end 98.868795 46.697195) (width 0.25) (layer "F.Cu") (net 12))
 (via (at 98.919596 46.697195) (size 0.8) (drill 0.4) (layers "F.Cu" "B.Cu") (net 12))
 (via (at 96.102501 43.930901) (size 0.8) (drill 0.4) (layers "F.Cu" "B.Cu") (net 12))
 (segment (start 114.2468 55.9816) (end 113.4848 55.2196) (width 0.25) (layer "B.Cu") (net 12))
 (segment (start 98.919596 46.697195) (end 100.624338 46.697195) (width 0.25) (layer "B.Cu") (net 12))
 (segment (start 100.624338 46.697195) (end 105.664 51.736857) (width 0.25) (layer "B.Cu") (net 12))
 (segment (start 105.664 53.8988) (end 106.9848 55.2196) (width 0.25) (layer "B.Cu") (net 12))
 (segment (start 105.664 51.736857) (end 105.664 53.8988) (width 0.25) (layer "B.Cu") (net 12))
 (segment (start 96.091402 43.942) (end 96.102501 43.930901) (width 0.25) (layer "B.Cu") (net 12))
 (segment (start 130.6068 53.15057) (end 127.77577 55.9816) (width 0.25) (layer "B.Cu") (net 12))
 (segment (start 130.6068 52.0192) (end 130.6068 53.15057) (width 0.25) (layer "B.Cu") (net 12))
 (segment (start 93.726 43.942) (end 96.091402 43.942) (width 0.25) (layer "B.Cu") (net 12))
 (segment (start 106.9848 55.2196) (end 113.4848 55.2196) (width 0.25) (layer "B.Cu") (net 12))
 (segment (start 127.77577 55.9816) (end 114.2468 55.9816) (width 0.25) (layer "B.Cu") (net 12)))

